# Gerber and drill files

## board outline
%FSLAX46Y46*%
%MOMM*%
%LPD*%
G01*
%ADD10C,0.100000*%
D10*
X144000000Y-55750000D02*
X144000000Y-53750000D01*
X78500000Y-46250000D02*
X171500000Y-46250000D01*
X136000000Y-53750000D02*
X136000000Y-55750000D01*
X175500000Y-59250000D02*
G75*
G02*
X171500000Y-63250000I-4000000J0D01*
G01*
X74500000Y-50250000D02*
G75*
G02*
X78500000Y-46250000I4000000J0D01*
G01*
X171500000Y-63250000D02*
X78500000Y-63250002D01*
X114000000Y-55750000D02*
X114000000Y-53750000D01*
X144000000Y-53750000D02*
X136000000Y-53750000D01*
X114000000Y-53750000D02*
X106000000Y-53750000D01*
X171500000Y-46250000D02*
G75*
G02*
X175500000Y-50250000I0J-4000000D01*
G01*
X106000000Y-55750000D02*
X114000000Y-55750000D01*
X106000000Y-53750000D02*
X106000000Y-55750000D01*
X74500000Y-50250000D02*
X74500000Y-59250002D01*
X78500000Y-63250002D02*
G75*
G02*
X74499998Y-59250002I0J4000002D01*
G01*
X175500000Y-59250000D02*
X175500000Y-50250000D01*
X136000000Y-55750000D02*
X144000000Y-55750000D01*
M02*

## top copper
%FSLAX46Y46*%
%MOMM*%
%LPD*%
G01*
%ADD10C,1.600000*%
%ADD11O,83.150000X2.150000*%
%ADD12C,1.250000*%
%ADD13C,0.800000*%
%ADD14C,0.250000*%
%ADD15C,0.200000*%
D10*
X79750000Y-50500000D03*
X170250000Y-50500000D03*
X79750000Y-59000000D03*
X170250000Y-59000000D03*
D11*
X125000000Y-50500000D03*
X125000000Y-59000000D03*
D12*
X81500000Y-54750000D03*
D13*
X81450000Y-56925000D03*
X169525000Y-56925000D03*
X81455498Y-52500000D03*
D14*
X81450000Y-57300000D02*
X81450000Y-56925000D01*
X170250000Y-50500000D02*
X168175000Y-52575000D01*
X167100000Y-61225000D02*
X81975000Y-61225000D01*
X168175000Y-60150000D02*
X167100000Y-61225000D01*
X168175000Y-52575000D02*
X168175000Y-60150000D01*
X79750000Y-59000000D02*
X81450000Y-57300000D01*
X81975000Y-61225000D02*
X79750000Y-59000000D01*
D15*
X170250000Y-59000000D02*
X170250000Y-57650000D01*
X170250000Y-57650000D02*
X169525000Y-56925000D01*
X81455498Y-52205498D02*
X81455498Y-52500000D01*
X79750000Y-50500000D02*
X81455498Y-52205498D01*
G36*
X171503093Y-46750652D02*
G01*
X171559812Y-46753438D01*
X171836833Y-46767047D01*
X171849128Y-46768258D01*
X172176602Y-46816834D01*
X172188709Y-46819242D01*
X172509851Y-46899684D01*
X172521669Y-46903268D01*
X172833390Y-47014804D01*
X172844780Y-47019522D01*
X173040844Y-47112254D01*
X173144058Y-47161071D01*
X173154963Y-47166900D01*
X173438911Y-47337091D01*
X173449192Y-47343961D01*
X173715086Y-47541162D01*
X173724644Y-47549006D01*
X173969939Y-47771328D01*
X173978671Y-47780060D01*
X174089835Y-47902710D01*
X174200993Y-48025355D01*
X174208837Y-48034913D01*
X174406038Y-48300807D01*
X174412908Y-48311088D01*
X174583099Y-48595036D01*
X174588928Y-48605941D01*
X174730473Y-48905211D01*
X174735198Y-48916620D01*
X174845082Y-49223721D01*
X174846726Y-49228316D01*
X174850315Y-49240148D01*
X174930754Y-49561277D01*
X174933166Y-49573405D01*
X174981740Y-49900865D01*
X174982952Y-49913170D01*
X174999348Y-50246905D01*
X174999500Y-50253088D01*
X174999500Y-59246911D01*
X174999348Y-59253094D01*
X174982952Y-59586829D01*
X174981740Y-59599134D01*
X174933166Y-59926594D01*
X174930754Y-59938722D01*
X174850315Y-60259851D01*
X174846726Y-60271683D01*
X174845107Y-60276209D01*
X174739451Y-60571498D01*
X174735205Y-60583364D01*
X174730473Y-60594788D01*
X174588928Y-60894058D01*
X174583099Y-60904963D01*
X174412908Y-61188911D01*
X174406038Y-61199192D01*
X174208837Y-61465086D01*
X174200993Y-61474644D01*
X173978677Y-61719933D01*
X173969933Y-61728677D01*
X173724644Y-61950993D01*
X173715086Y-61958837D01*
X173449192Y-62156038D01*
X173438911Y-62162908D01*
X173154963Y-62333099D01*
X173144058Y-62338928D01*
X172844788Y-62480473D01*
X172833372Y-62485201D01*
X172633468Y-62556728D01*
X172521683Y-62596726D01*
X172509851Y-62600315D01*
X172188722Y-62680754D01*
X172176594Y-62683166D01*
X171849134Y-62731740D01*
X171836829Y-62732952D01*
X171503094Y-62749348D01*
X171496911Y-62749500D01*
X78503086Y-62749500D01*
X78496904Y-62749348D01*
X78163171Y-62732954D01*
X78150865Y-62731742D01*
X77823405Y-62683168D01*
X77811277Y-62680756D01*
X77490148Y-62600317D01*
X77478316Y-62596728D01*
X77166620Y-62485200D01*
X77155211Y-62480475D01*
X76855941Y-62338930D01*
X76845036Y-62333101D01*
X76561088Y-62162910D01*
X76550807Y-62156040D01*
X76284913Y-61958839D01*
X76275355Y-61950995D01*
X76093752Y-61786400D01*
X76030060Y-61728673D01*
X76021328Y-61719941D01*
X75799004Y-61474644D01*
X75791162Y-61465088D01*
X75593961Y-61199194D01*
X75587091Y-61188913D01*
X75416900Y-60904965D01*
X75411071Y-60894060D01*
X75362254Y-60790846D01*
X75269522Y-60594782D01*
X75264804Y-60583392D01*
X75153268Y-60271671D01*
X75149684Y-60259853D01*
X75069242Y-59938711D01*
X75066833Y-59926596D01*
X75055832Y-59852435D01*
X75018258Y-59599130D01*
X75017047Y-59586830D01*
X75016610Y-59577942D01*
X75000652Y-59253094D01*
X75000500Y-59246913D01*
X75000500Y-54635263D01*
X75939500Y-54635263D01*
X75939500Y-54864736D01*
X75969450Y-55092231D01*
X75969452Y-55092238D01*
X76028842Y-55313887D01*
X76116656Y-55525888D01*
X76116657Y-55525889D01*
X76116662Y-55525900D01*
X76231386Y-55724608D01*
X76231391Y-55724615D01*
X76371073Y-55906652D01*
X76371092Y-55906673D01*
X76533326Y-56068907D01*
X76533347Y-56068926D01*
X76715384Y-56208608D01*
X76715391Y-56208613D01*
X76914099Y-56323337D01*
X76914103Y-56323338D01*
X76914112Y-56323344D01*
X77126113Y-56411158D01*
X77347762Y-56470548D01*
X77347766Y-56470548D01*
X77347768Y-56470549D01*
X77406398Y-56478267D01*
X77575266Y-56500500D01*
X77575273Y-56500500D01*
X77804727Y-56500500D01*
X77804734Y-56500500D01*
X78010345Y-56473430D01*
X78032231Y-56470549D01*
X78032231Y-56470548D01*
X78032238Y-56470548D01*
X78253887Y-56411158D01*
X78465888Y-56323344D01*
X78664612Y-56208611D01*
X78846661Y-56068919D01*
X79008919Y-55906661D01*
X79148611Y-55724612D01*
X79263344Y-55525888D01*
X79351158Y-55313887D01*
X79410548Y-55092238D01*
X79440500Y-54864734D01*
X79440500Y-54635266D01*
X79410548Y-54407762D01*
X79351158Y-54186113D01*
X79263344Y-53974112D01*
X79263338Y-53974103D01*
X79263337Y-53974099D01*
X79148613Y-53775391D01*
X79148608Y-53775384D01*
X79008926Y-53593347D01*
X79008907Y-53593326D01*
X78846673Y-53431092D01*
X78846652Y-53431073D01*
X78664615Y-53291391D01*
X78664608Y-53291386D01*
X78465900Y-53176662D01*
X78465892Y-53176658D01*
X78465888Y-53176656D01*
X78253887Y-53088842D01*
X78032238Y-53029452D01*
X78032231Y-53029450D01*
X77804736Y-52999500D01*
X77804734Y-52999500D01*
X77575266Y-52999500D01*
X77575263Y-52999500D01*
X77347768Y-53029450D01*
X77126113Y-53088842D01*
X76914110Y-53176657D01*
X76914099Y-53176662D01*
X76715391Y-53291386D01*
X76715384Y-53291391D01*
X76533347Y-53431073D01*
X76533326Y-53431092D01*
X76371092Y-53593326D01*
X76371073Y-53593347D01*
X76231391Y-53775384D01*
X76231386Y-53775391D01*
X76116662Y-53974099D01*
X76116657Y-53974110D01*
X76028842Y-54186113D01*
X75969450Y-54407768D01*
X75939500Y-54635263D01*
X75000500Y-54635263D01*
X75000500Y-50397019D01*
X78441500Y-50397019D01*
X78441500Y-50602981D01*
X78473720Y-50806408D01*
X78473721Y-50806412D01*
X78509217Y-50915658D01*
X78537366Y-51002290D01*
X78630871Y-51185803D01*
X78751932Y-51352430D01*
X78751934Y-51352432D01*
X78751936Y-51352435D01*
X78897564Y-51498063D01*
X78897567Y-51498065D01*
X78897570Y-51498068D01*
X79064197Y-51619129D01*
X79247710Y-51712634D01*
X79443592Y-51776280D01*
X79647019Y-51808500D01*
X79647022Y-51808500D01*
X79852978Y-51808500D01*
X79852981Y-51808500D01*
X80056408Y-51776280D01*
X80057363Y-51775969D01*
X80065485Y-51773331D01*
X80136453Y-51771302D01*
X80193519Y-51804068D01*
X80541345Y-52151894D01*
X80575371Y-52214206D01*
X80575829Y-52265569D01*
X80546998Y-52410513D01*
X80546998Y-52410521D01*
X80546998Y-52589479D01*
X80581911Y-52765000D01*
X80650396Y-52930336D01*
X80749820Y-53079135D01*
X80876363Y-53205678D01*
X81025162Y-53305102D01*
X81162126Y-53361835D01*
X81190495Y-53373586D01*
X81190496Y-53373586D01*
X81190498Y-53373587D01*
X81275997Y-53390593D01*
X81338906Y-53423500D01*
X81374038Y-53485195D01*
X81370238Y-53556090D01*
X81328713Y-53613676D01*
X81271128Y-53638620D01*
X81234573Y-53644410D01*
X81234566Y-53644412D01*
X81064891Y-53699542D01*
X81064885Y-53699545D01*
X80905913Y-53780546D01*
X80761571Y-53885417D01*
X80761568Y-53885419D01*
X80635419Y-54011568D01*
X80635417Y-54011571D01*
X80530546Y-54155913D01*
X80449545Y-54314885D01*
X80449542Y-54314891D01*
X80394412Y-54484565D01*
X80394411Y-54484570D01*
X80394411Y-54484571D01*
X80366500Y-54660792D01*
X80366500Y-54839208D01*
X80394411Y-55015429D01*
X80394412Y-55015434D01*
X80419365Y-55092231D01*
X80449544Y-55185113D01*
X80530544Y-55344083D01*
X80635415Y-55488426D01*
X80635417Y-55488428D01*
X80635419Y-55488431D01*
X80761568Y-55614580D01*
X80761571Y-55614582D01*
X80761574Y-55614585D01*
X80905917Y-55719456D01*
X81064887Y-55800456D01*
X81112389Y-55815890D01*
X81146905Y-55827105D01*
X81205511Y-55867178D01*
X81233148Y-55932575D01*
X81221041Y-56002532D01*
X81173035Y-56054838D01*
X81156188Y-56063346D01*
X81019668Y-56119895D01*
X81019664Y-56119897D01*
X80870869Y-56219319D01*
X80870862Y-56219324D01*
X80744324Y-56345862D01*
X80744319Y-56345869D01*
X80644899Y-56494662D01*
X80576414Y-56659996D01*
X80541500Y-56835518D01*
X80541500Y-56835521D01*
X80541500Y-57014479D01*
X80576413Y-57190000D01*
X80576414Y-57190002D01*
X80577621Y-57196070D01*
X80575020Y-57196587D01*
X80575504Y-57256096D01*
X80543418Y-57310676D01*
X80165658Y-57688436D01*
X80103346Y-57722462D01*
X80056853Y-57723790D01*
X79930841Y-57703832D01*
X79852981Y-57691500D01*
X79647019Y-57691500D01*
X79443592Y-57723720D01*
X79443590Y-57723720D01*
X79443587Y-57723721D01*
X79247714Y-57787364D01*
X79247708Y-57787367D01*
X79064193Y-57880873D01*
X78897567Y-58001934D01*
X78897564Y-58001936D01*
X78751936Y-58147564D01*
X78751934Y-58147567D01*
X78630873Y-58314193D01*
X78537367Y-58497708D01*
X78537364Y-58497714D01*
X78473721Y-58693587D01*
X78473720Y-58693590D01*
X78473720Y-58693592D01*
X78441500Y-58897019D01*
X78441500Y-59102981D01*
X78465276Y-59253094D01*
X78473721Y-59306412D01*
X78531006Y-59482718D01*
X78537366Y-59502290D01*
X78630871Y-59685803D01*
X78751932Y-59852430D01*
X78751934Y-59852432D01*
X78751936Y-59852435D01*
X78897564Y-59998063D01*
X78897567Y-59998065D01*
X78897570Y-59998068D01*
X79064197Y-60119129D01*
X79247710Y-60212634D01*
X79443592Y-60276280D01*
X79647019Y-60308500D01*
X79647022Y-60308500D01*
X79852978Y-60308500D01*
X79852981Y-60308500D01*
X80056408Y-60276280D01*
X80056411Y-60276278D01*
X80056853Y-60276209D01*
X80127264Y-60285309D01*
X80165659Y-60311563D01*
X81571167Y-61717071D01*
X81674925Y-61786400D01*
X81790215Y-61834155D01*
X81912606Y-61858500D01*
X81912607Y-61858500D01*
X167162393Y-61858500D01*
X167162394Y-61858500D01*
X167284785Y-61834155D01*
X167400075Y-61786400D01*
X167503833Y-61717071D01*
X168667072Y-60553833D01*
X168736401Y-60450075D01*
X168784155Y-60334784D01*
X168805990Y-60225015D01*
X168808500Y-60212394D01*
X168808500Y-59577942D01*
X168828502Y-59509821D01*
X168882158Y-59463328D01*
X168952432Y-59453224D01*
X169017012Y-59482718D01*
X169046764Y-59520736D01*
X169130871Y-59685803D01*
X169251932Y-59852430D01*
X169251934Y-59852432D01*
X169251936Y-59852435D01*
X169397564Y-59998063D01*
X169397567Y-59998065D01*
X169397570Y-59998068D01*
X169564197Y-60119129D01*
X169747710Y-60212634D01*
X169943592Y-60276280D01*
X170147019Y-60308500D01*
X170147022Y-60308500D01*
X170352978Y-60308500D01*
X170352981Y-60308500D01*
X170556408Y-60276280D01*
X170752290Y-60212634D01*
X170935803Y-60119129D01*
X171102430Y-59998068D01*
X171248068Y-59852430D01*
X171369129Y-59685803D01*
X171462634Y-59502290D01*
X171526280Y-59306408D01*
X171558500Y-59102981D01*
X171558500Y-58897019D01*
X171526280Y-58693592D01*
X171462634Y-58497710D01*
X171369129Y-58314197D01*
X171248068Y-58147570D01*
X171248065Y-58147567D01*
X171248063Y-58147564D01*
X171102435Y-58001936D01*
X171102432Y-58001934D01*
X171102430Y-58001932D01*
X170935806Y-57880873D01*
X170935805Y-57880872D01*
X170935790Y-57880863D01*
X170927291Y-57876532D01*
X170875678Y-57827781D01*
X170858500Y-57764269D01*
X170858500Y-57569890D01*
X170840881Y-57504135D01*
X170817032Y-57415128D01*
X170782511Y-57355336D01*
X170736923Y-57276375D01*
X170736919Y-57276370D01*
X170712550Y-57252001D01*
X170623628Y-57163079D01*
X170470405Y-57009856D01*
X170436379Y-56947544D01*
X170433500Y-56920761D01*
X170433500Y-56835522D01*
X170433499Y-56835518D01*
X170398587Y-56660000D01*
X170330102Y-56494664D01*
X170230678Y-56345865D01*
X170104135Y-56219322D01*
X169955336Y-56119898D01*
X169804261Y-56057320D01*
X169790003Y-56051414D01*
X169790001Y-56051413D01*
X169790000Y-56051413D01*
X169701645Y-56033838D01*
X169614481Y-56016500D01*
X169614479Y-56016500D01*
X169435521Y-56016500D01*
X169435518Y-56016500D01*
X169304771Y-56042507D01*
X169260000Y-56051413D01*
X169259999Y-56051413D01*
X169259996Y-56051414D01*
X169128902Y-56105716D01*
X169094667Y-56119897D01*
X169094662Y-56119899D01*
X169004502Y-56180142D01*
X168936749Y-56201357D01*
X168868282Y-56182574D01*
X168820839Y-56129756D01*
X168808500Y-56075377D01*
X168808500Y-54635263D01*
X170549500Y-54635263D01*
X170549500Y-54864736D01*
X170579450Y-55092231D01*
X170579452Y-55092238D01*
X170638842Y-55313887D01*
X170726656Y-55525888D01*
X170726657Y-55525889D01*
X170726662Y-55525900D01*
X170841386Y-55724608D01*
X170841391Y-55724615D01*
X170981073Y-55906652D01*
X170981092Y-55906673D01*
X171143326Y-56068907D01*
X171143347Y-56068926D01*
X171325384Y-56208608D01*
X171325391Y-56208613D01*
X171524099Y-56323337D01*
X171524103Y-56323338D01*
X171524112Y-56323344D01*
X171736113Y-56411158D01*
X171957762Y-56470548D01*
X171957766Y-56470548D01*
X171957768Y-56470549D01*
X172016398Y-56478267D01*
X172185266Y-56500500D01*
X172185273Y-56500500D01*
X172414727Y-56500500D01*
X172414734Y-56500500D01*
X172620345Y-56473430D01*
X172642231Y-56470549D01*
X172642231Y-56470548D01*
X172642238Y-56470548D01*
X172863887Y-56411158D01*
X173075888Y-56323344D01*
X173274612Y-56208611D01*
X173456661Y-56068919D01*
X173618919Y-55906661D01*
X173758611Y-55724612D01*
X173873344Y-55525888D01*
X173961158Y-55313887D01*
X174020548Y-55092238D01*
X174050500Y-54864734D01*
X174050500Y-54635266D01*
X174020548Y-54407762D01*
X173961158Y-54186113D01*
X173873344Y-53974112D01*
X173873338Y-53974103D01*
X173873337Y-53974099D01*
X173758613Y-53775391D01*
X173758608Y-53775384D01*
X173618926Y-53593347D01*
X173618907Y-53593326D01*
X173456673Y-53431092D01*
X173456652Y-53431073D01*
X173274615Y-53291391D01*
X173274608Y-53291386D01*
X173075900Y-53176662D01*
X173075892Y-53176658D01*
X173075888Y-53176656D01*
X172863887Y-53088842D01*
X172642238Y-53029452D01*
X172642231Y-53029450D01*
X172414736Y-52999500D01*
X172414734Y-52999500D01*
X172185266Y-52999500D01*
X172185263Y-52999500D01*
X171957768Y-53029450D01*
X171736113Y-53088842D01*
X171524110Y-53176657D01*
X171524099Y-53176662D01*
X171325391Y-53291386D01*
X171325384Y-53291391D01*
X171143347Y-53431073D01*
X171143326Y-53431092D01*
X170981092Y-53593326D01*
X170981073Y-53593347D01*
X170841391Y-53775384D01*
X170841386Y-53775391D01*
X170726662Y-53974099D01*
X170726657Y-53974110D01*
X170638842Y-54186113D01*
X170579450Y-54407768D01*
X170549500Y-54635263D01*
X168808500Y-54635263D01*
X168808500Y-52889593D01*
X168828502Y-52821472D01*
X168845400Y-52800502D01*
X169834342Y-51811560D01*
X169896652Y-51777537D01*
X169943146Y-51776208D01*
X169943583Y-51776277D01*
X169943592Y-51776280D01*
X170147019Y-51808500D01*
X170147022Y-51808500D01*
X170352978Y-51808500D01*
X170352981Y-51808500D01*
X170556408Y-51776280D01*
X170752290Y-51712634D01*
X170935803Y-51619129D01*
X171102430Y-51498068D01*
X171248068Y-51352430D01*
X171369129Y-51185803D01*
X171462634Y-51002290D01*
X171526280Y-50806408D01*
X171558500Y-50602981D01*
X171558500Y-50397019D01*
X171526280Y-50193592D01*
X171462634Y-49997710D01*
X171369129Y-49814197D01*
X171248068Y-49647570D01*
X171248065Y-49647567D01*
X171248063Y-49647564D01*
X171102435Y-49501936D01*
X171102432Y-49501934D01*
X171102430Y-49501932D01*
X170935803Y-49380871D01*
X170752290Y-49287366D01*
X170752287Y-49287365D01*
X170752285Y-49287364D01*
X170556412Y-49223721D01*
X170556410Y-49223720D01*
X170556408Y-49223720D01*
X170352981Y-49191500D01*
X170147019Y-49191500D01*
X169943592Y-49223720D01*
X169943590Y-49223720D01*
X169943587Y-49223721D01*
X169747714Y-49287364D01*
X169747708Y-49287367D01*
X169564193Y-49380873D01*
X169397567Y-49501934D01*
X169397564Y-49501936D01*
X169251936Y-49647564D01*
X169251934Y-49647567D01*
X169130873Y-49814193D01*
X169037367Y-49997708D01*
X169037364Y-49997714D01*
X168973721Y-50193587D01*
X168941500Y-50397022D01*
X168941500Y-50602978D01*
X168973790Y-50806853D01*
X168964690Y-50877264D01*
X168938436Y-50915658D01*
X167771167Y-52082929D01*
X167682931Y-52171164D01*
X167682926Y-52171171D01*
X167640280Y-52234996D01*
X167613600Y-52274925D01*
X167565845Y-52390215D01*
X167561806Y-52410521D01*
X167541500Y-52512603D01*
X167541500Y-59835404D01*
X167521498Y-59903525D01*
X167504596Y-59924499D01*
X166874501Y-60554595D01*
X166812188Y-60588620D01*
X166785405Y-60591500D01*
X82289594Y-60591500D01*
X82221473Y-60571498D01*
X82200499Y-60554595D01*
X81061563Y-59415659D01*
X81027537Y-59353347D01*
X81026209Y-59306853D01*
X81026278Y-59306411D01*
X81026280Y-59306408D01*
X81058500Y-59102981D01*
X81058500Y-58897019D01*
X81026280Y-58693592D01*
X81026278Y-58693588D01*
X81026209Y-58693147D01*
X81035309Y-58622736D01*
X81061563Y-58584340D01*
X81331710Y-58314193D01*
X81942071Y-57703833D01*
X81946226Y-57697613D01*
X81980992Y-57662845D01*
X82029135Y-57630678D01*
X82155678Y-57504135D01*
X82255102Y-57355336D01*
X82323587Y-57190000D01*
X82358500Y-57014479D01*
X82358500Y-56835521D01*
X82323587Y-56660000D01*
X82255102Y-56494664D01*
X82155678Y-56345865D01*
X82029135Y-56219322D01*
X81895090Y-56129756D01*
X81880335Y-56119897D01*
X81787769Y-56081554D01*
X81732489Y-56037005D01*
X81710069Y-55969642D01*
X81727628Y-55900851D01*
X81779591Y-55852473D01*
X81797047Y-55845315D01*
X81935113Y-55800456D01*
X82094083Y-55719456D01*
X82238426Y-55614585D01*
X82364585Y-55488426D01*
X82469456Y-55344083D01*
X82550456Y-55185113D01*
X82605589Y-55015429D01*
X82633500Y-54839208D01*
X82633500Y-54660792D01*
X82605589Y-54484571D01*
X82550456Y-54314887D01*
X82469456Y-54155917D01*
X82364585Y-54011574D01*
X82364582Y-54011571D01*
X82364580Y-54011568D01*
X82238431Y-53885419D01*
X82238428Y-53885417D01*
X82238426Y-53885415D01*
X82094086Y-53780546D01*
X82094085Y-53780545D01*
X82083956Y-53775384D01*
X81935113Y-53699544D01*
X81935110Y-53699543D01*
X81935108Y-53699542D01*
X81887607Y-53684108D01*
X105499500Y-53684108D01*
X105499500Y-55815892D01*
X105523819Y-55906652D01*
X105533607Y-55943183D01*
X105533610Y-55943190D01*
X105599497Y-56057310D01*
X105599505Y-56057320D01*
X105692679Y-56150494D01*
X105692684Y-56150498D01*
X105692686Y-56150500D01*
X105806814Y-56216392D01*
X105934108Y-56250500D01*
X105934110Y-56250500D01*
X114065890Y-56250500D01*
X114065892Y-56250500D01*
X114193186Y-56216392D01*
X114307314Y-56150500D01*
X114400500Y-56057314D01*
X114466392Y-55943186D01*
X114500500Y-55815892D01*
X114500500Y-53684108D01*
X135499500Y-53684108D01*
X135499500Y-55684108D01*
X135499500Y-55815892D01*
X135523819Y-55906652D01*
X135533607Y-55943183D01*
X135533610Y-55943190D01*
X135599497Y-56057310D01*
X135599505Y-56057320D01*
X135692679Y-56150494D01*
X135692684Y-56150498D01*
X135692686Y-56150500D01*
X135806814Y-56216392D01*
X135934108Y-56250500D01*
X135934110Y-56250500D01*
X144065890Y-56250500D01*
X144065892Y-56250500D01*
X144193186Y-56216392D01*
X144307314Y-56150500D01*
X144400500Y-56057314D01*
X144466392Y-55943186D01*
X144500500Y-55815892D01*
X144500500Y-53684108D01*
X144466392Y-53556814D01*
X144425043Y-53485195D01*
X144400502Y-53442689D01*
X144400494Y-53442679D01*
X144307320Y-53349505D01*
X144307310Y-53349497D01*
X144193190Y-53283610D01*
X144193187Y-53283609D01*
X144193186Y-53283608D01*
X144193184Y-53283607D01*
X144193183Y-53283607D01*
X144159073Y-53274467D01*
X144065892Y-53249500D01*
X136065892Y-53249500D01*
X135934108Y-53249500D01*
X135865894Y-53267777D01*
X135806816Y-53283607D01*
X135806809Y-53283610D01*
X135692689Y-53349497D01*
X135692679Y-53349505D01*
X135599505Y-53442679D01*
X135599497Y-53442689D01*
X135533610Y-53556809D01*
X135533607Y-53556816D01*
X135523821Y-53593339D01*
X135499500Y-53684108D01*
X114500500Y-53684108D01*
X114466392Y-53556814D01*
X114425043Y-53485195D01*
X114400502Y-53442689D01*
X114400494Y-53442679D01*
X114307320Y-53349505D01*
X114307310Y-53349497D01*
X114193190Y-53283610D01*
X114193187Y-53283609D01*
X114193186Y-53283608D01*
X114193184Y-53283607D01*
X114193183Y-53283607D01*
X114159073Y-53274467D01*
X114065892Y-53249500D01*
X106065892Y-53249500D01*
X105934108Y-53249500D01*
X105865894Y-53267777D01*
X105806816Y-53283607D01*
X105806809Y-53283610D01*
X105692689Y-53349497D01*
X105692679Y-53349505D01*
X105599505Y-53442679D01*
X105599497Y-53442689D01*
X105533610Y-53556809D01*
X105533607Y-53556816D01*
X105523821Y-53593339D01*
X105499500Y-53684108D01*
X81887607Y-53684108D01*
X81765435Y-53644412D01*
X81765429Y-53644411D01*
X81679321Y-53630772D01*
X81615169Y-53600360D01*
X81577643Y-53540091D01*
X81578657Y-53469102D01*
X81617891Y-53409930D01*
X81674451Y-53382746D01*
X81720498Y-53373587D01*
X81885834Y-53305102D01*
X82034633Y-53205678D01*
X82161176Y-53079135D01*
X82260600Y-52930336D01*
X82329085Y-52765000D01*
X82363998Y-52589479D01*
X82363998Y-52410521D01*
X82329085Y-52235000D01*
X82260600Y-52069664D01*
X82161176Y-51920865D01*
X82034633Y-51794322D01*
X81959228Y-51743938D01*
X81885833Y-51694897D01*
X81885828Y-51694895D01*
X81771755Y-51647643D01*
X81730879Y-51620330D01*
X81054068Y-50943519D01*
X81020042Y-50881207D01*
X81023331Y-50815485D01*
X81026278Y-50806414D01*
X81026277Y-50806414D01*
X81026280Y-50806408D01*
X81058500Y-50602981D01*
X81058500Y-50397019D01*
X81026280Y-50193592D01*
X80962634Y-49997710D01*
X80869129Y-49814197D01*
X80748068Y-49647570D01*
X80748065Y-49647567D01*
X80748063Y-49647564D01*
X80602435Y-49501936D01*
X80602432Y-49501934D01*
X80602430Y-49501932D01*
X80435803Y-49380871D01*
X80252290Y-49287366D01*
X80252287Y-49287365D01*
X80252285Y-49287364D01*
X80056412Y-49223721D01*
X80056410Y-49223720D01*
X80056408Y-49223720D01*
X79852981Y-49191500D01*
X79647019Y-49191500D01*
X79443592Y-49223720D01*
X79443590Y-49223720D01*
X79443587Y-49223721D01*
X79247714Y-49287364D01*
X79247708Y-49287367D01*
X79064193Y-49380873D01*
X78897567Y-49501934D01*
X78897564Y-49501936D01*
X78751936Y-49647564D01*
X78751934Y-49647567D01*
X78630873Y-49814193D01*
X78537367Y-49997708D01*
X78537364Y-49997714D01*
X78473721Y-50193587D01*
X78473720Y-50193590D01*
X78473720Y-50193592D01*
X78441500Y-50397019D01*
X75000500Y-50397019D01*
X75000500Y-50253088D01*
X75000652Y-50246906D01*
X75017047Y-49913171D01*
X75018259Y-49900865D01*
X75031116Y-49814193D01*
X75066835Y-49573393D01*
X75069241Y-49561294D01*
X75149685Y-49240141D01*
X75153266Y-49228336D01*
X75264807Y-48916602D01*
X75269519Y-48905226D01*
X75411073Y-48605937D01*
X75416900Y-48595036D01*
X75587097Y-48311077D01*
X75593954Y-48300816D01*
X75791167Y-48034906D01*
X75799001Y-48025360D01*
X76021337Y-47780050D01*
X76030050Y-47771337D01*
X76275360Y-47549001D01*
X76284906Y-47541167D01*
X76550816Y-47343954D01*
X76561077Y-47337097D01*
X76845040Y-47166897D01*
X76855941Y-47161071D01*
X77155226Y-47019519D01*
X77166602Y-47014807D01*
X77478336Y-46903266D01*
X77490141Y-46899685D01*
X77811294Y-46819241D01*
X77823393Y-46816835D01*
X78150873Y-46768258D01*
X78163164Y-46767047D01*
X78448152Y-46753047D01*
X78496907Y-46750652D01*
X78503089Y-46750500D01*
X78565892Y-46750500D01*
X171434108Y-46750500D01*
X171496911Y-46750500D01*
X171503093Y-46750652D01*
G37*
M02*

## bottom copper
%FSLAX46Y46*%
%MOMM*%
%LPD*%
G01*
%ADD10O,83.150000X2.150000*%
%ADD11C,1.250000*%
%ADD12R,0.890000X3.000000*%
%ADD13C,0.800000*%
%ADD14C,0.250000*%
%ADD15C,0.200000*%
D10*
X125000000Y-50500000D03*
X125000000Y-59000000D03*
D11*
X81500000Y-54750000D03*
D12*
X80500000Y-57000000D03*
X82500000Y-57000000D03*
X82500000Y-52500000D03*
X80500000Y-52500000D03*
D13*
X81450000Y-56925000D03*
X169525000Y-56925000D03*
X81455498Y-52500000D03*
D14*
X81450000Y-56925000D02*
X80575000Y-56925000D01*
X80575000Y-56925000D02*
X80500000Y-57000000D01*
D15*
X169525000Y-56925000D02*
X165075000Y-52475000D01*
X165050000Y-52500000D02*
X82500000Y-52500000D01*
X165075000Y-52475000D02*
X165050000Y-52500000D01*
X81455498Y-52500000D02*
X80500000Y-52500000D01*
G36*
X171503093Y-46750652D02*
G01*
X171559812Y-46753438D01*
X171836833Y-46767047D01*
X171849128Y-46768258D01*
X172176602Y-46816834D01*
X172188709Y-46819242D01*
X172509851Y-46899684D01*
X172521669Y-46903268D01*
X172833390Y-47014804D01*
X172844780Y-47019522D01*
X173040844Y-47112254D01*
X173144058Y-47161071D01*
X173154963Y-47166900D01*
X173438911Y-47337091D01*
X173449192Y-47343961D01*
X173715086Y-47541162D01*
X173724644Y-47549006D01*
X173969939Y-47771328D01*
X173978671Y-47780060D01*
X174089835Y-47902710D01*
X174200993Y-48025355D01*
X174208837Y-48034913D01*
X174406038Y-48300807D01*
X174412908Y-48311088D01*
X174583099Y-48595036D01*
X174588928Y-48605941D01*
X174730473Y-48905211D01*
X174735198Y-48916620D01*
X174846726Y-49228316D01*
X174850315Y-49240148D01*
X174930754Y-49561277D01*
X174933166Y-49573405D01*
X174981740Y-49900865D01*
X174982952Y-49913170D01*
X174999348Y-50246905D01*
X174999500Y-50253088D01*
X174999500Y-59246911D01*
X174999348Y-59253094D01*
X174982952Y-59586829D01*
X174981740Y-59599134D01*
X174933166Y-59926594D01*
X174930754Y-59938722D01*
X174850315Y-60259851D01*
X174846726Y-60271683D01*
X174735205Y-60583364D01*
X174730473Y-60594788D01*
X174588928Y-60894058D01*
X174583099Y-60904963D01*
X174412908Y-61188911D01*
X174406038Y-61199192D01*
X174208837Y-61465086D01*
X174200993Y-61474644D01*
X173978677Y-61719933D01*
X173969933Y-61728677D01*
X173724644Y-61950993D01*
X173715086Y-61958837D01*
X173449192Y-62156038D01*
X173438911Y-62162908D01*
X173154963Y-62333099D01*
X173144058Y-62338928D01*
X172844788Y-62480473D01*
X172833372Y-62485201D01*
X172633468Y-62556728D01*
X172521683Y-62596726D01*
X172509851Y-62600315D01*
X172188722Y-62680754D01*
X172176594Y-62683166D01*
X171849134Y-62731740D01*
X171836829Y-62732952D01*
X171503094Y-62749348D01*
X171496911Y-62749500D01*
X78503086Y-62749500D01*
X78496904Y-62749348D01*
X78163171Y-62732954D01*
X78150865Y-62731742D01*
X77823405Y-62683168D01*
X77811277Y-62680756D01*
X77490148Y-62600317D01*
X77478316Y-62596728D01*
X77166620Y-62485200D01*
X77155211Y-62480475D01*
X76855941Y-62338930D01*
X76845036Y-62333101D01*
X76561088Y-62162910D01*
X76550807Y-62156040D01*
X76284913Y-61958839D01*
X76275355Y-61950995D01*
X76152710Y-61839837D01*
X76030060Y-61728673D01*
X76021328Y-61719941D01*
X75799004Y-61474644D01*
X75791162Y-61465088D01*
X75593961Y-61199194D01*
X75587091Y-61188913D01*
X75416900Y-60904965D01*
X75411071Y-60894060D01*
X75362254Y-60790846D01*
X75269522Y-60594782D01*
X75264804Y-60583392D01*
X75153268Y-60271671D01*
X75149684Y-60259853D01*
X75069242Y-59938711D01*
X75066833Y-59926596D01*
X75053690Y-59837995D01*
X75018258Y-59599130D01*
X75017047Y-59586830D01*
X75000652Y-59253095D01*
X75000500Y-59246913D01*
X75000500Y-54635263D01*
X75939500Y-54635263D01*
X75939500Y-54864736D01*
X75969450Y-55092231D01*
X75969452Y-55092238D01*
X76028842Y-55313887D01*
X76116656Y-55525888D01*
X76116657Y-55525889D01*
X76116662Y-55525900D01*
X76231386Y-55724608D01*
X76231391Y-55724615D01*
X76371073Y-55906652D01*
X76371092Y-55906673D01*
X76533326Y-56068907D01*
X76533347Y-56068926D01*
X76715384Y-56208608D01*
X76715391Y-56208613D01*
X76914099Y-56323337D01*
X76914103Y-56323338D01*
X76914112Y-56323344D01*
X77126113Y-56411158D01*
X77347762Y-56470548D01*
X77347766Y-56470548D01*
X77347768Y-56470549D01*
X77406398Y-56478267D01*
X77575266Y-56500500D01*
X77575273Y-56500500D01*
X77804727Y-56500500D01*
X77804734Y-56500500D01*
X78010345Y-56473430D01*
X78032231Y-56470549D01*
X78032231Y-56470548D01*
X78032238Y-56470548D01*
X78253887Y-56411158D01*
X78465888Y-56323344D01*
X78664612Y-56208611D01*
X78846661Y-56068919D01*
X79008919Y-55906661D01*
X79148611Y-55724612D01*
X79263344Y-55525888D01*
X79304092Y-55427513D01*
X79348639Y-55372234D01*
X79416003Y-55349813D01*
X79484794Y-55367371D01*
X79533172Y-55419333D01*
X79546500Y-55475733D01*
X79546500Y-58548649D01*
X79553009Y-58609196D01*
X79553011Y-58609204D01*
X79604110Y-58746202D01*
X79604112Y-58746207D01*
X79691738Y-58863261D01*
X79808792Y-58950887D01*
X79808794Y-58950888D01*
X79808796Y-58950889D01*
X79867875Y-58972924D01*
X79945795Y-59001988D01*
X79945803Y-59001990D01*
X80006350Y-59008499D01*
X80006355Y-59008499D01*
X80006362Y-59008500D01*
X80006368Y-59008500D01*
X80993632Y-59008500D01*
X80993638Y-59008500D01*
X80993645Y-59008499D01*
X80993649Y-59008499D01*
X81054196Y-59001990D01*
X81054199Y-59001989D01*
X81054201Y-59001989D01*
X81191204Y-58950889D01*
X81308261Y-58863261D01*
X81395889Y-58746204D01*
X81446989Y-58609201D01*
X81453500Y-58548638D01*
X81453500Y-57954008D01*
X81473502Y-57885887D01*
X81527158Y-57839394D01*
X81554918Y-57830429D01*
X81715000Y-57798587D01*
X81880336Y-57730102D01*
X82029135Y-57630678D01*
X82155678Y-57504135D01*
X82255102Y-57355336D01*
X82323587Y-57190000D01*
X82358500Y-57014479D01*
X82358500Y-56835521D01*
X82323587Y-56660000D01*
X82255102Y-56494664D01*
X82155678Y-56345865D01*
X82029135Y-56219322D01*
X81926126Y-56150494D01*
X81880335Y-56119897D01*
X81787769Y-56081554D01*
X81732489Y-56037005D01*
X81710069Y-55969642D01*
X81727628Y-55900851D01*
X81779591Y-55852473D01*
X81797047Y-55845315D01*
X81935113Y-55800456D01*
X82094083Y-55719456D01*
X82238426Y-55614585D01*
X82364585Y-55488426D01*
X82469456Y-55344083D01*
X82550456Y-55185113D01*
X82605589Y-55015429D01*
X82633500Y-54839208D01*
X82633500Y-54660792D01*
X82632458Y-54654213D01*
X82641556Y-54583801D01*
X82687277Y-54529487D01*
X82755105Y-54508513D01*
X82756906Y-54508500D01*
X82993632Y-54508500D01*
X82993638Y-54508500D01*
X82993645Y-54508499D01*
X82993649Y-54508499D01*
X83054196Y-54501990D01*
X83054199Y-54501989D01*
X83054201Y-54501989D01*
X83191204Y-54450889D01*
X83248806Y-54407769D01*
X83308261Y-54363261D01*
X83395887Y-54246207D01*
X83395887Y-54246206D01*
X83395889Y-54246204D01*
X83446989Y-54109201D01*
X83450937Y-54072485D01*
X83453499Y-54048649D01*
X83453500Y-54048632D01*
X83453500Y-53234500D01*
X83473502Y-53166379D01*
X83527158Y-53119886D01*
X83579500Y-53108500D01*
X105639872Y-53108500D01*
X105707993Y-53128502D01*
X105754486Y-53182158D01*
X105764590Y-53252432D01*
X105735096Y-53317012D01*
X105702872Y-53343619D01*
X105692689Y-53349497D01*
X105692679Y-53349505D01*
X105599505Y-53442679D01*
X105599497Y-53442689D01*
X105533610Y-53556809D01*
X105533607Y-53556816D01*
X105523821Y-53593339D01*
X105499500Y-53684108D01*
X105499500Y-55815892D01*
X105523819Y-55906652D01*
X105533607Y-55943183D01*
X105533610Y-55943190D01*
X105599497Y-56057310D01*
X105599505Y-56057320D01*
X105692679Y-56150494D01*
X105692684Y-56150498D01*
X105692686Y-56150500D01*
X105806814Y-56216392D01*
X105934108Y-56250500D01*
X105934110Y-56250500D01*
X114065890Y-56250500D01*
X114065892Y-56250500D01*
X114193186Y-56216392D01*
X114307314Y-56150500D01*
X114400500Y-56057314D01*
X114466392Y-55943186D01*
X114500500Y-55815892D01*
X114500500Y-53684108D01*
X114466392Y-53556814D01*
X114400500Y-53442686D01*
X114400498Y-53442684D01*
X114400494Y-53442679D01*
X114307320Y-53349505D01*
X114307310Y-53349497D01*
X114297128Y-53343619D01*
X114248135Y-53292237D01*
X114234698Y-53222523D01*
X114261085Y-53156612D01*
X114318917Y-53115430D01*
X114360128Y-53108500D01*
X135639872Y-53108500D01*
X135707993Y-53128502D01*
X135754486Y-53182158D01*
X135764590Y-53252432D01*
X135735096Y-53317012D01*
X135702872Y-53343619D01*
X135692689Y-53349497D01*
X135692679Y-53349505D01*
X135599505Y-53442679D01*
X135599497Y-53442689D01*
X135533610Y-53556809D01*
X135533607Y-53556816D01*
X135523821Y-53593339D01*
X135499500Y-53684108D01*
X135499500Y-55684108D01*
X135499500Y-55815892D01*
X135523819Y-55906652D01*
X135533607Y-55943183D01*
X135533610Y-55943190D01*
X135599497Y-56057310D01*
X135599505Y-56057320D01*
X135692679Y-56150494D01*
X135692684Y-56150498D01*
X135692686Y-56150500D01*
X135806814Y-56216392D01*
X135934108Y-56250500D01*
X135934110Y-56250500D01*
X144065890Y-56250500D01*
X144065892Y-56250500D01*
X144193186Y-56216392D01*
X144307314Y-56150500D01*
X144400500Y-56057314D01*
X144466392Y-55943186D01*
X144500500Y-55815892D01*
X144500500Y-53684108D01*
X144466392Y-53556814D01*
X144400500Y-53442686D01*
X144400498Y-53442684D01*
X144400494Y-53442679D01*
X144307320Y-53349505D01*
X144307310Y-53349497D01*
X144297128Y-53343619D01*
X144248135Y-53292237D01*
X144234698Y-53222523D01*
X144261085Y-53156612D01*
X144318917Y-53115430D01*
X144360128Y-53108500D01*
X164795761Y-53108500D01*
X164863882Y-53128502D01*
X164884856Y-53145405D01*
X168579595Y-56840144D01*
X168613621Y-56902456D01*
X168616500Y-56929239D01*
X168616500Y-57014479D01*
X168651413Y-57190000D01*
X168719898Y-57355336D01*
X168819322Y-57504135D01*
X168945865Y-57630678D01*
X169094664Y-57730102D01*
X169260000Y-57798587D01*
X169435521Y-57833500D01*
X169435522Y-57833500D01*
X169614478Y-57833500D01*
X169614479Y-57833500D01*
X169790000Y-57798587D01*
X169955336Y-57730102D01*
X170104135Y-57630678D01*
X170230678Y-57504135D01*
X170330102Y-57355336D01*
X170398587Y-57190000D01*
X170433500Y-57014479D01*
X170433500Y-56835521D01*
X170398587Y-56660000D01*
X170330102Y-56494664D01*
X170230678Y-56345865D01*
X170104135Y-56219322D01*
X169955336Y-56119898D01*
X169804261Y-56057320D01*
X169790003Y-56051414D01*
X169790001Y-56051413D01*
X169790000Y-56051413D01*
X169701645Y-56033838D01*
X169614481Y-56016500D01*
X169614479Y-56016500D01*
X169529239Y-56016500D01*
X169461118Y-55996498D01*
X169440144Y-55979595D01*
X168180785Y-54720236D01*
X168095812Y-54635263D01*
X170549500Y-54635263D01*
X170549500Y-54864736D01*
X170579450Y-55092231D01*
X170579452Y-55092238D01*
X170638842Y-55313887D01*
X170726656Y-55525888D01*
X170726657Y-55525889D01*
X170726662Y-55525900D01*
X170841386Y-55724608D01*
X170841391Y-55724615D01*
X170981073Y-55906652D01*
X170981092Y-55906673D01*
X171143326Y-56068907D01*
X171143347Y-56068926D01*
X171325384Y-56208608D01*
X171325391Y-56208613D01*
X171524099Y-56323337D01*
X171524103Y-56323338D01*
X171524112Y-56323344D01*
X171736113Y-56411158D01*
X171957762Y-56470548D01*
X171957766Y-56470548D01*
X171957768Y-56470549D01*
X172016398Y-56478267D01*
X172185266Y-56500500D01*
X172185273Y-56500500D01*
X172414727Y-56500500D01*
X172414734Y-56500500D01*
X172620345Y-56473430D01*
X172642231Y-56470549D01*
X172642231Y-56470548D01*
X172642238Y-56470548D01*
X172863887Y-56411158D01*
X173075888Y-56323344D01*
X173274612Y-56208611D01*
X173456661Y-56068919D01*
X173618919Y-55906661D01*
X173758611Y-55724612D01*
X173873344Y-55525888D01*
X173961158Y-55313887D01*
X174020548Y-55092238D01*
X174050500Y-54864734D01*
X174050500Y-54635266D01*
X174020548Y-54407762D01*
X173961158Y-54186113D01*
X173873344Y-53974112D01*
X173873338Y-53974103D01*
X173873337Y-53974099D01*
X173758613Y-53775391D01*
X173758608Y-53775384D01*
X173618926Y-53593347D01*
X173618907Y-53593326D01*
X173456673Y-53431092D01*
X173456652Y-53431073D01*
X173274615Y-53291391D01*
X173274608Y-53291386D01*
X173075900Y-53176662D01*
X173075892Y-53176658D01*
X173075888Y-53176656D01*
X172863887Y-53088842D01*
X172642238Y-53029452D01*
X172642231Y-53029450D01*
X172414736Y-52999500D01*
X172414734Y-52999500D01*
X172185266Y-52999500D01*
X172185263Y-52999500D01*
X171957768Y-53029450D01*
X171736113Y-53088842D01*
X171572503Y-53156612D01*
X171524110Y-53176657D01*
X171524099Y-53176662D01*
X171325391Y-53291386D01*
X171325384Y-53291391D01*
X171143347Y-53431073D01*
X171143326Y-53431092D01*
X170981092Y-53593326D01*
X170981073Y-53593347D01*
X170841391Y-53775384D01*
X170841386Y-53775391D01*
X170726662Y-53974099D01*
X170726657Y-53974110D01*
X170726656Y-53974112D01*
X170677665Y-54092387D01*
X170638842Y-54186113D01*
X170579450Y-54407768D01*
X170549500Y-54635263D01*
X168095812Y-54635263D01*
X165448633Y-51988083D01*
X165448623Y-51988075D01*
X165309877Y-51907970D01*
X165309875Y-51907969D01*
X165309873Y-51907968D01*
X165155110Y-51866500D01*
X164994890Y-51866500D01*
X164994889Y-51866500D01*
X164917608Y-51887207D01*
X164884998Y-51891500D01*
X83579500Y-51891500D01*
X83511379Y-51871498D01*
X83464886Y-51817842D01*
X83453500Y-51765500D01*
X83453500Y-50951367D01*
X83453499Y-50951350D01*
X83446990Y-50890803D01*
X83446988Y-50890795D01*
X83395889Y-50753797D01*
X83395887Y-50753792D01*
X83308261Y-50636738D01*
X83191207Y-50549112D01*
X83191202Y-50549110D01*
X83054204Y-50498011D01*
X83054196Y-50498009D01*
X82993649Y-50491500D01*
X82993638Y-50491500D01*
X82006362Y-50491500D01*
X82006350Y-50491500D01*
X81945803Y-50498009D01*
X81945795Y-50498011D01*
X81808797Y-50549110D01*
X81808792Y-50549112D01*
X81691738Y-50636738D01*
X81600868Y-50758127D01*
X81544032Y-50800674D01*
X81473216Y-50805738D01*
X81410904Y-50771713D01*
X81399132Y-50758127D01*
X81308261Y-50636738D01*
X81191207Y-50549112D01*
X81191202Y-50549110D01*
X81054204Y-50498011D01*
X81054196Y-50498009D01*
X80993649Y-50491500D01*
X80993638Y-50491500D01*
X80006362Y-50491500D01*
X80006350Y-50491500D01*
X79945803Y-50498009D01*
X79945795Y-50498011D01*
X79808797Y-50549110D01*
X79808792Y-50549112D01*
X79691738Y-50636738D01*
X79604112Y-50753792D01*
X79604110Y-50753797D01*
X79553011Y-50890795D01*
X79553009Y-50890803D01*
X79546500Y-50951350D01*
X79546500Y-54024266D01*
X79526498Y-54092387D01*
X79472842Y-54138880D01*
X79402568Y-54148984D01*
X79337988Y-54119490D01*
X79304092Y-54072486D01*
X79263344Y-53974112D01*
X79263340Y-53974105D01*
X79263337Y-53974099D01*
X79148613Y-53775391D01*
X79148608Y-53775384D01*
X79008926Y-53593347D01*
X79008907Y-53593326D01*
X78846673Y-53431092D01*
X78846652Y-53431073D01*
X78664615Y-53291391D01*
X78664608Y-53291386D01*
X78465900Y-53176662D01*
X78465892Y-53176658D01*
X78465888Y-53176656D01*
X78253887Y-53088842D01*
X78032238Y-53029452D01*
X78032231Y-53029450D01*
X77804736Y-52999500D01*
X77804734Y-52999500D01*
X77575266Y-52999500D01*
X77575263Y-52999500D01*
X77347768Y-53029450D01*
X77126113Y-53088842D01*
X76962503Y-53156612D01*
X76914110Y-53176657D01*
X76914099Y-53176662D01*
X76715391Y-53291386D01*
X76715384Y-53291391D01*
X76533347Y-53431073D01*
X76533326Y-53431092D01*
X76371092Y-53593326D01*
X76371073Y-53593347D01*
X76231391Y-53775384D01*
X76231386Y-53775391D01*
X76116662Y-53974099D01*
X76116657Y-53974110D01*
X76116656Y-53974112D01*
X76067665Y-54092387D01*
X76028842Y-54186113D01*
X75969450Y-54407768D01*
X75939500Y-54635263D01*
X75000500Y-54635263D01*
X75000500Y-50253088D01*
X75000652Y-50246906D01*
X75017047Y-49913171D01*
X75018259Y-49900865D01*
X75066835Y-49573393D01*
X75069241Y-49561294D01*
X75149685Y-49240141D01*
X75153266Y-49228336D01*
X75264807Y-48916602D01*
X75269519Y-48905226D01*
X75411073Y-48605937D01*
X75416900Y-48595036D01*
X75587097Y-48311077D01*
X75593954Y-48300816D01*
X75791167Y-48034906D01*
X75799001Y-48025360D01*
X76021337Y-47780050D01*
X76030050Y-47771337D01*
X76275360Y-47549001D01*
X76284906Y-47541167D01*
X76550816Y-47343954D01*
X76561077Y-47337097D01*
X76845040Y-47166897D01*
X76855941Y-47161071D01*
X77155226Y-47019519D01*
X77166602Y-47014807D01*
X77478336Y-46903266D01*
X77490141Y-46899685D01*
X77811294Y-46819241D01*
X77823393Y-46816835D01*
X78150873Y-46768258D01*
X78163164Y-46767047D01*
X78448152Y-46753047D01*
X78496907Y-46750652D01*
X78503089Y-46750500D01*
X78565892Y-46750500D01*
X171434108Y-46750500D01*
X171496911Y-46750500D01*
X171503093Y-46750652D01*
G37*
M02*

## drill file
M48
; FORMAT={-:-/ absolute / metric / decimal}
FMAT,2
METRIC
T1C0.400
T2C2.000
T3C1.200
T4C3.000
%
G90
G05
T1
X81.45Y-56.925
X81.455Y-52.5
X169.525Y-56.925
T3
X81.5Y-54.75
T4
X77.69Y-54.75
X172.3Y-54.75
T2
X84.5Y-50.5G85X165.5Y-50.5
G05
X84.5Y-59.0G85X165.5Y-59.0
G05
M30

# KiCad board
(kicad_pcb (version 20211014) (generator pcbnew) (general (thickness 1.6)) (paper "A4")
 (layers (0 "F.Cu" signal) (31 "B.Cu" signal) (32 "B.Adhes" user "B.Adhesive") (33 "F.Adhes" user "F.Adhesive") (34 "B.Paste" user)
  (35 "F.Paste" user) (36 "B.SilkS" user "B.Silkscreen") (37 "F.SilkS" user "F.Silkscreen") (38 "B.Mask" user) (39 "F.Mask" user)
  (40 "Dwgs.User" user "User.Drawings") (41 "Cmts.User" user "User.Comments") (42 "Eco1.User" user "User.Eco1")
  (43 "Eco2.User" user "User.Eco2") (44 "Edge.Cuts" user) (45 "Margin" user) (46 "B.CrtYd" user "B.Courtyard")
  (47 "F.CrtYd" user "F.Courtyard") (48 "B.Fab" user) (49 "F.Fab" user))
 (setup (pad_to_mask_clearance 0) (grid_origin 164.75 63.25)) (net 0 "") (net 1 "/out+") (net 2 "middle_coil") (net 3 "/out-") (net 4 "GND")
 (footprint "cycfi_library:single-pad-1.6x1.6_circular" (layer "F.Cu") (at 79.75 50.5)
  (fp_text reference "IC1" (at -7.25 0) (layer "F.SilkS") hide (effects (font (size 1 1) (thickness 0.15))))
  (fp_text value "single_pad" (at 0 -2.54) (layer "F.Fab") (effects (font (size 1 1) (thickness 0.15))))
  (pad "1" smd circle (at 0 0) (size 1.6 1.6) (layers "F.Cu" "F.Paste" "F.Mask") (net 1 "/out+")))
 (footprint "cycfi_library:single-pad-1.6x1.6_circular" (layer "F.Cu") (at 170.25 50.5)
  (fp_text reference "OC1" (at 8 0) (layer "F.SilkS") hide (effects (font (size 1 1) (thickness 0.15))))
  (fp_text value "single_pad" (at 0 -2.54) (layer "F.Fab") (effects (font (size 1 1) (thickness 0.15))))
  (pad "1" smd circle (at 0 0) (size 1.6 1.6) (layers "F.Cu" "F.Paste" "F.Mask") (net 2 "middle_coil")))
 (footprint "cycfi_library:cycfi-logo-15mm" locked (layer "F.Cu") (at 124.75 54.75)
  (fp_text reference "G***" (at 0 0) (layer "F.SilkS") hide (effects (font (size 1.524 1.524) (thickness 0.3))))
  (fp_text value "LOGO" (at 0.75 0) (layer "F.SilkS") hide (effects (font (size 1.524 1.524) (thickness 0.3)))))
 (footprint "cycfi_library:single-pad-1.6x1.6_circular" (layer "F.Cu") (at 79.75 59)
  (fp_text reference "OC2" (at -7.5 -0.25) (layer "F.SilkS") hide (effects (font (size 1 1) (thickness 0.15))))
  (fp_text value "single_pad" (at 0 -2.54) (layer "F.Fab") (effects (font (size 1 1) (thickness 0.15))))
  (pad "1" smd circle (at 0 0) (size 1.6 1.6) (layers "F.Cu" "F.Paste" "F.Mask") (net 2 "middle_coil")))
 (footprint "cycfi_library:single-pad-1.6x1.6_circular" (layer "F.Cu") (at 170.25 59)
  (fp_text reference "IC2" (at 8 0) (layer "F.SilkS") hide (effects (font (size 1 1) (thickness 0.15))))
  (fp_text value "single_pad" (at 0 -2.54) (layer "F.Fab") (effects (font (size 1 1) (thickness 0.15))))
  (pad "1" smd circle (at 0 0) (size 1.6 1.6) (layers "F.Cu" "F.Paste" "F.Mask") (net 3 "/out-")))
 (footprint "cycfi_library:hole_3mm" (layer "F.Cu") (at 172.3 54.75 180)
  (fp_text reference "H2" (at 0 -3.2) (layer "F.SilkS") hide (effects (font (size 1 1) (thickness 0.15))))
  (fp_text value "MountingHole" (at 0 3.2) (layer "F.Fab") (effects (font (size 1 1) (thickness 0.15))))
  (pad "" np_thru_hole circle (at 0 0 180) (size 3 3) (drill 3) (layers F&B.Cu *.Mask)))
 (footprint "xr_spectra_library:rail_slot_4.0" (layer "F.Cu") (at 125 50.5)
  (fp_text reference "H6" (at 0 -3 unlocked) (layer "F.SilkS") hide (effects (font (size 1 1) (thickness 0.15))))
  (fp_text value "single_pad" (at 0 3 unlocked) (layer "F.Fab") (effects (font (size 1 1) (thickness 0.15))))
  (pad "1" thru_hole oval (at 0 0) (size 83.15 2.15) (drill oval 83 2) (layers *.Cu *.Mask) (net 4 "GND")))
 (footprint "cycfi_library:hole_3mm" (layer "F.Cu") (at 77.69 54.75 180)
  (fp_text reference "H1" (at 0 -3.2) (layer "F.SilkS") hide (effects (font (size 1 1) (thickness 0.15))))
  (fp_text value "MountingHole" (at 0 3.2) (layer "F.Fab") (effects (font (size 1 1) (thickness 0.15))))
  (pad "" np_thru_hole circle (at 0 0 180) (size 3 3) (drill 3) (layers F&B.Cu *.Mask)))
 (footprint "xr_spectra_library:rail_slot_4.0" (layer "F.Cu") (at 125 59)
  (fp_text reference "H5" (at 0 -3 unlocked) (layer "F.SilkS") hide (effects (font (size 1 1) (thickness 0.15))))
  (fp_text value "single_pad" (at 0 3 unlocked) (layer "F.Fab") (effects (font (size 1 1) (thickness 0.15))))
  (pad "1" thru_hole oval (at 0 0) (size 83.15 2.15) (drill oval 83 2) (layers *.Cu *.Mask) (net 4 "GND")))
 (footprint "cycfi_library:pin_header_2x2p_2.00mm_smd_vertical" (layer "B.Cu") (at 81.5 54.75 -90)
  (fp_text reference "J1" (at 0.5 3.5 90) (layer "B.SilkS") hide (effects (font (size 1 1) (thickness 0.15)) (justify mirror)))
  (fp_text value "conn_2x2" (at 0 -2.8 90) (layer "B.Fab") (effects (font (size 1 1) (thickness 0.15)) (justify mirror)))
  (pad "" np_thru_hole circle (at 0 0 270) (size 1.25 1.25) (drill 1.2) (layers F&B.Cu *.Mask))
  (pad "1" smd rect (at 2.25 1 270) (size 3 0.89) (layers "B.Cu" "B.Paste" "B.Mask") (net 2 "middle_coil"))
  (pad "2" smd rect (at 2.25 -1 270) (size 3 0.89) (layers "B.Cu" "B.Paste" "B.Mask") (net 4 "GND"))
  (pad "3" smd rect (at -2.25 -1 270) (size 3 0.89) (layers "B.Cu" "B.Paste" "B.Mask") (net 3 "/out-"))
  (pad "4" smd rect (at -2.25 1 270) (size 3 0.89) (layers "B.Cu" "B.Paste" "B.Mask") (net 1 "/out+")))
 (gr_line (start 144 55.75) (end 144 53.75) (layer "Edge.Cuts") (width 0.1))
 (gr_line (start 78.5 46.25) (end 171.5 46.25) (layer "Edge.Cuts") (width 0.1))
 (gr_line (start 136 53.75) (end 136 55.75) (layer "Edge.Cuts") (width 0.1))
 (gr_arc (start 175.5 59.25) (mid 174.328427 62.078427) (end 171.5 63.25) (layer "Edge.Cuts") (width 0.1))
 (gr_arc (start 74.5 50.25) (mid 75.671573 47.421573) (end 78.5 46.25) (layer "Edge.Cuts") (width 0.1))
 (gr_line (start 171.5 63.25) (end 78.5 63.250002) (layer "Edge.Cuts") (width 0.1))
 (gr_line (start 114 55.75) (end 114 53.75) (layer "Edge.Cuts") (width 0.1))
 (gr_line (start 144 53.75) (end 136 53.75) (layer "Edge.Cuts") (width 0.1))
 (gr_line (start 114 53.75) (end 106 53.75) (layer "Edge.Cuts") (width 0.1))
 (gr_arc (start 171.5 46.25) (mid 174.328427 47.421573) (end 175.5 50.25) (layer "Edge.Cuts") (width 0.1))
 (gr_line (start 106 55.75) (end 114 55.75) (layer "Edge.Cuts") (width 0.1))
 (gr_line (start 106 53.75) (end 106 55.75) (layer "Edge.Cuts") (width 0.1))
 (gr_line (start 74.5 50.25) (end 74.5 59.250002) (layer "Edge.Cuts") (width 0.1))
 (gr_arc (start 78.5 63.250002) (mid 75.671573 62.078429) (end 74.5 59.250002) (layer "Edge.Cuts") (width 0.1))
 (gr_line (start 175.5 59.25) (end 175.5 50.25) (layer "Edge.Cuts") (width 0.1))
 (gr_line (start 136 55.75) (end 144 55.75) (layer "Edge.Cuts") (width 0.1))
 (segment (start 81.45 57.3) (end 81.45 56.925) (width 0.25) (layer "F.Cu") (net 2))
 (segment (start 170.25 50.5) (end 168.175 52.575) (width 0.25) (layer "F.Cu") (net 2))
 (segment (start 167.1 61.225) (end 81.975 61.225) (width 0.25) (layer "F.Cu") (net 2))
 (segment (start 168.175 60.15) (end 167.1 61.225) (width 0.25) (layer "F.Cu") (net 2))
 (segment (start 168.175 52.575) (end 168.175 60.15) (width 0.25) (layer "F.Cu") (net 2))
 (segment (start 79.75 59) (end 81.45 57.3) (width 0.25) (layer "F.Cu") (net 2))
 (segment (start 81.975 61.225) (end 79.75 59) (width 0.25) (layer "F.Cu") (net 2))
 (via (at 81.45 56.925) (size 0.8) (drill 0.4) (layers "F.Cu" "B.Cu") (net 2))
 (segment (start 81.45 56.925) (end 80.575 56.925) (width 0.25) (layer "B.Cu") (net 2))
 (segment (start 80.575 56.925) (end 80.5 57) (width 0.25) (layer "B.Cu") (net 2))
 (segment (start 170.25 59) (end 170.25 57.65) (width 0.2) (layer "F.Cu") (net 3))
 (segment (start 170.25 57.65) (end 169.525 56.925) (width 0.2) (layer "F.Cu") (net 3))
 (via (at 169.525 56.925) (size 0.8) (drill 0.4) (layers "F.Cu" "B.Cu") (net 3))
 (segment (start 169.525 56.925) (end 165.075 52.475) (width 0.2) (layer "B.Cu") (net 3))
 (segment (start 165.05 52.5) (end 82.5 52.5) (width 0.2) (layer "B.Cu") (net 3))
 (segment (start 165.075 52.475) (end 165.05 52.5) (width 0.2) (layer "B.Cu") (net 3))
 (segment (start 81.455498 52.205498) (end 81.455498 52.5) (width 0.2) (layer "F.Cu") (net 1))
 (segment (start 79.75 50.5) (end 81.455498 52.205498) (width 0.2) (layer "F.Cu") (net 1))
 (via (at 81.455498 52.5) (size 0.8) (drill 0.4) (layers "F.Cu" "B.Cu") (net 1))
 (segment (start 81.455498 52.5) (end 80.5 52.5) (width 0.2) (layer "B.Cu") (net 1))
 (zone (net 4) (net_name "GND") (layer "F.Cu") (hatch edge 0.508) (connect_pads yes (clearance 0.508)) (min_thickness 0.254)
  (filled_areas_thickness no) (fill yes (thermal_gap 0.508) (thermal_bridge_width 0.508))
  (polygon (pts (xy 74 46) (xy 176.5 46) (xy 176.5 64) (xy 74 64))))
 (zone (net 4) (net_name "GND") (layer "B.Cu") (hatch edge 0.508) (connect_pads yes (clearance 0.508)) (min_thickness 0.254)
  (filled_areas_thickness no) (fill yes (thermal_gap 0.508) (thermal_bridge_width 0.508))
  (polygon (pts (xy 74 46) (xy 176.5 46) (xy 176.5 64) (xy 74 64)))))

